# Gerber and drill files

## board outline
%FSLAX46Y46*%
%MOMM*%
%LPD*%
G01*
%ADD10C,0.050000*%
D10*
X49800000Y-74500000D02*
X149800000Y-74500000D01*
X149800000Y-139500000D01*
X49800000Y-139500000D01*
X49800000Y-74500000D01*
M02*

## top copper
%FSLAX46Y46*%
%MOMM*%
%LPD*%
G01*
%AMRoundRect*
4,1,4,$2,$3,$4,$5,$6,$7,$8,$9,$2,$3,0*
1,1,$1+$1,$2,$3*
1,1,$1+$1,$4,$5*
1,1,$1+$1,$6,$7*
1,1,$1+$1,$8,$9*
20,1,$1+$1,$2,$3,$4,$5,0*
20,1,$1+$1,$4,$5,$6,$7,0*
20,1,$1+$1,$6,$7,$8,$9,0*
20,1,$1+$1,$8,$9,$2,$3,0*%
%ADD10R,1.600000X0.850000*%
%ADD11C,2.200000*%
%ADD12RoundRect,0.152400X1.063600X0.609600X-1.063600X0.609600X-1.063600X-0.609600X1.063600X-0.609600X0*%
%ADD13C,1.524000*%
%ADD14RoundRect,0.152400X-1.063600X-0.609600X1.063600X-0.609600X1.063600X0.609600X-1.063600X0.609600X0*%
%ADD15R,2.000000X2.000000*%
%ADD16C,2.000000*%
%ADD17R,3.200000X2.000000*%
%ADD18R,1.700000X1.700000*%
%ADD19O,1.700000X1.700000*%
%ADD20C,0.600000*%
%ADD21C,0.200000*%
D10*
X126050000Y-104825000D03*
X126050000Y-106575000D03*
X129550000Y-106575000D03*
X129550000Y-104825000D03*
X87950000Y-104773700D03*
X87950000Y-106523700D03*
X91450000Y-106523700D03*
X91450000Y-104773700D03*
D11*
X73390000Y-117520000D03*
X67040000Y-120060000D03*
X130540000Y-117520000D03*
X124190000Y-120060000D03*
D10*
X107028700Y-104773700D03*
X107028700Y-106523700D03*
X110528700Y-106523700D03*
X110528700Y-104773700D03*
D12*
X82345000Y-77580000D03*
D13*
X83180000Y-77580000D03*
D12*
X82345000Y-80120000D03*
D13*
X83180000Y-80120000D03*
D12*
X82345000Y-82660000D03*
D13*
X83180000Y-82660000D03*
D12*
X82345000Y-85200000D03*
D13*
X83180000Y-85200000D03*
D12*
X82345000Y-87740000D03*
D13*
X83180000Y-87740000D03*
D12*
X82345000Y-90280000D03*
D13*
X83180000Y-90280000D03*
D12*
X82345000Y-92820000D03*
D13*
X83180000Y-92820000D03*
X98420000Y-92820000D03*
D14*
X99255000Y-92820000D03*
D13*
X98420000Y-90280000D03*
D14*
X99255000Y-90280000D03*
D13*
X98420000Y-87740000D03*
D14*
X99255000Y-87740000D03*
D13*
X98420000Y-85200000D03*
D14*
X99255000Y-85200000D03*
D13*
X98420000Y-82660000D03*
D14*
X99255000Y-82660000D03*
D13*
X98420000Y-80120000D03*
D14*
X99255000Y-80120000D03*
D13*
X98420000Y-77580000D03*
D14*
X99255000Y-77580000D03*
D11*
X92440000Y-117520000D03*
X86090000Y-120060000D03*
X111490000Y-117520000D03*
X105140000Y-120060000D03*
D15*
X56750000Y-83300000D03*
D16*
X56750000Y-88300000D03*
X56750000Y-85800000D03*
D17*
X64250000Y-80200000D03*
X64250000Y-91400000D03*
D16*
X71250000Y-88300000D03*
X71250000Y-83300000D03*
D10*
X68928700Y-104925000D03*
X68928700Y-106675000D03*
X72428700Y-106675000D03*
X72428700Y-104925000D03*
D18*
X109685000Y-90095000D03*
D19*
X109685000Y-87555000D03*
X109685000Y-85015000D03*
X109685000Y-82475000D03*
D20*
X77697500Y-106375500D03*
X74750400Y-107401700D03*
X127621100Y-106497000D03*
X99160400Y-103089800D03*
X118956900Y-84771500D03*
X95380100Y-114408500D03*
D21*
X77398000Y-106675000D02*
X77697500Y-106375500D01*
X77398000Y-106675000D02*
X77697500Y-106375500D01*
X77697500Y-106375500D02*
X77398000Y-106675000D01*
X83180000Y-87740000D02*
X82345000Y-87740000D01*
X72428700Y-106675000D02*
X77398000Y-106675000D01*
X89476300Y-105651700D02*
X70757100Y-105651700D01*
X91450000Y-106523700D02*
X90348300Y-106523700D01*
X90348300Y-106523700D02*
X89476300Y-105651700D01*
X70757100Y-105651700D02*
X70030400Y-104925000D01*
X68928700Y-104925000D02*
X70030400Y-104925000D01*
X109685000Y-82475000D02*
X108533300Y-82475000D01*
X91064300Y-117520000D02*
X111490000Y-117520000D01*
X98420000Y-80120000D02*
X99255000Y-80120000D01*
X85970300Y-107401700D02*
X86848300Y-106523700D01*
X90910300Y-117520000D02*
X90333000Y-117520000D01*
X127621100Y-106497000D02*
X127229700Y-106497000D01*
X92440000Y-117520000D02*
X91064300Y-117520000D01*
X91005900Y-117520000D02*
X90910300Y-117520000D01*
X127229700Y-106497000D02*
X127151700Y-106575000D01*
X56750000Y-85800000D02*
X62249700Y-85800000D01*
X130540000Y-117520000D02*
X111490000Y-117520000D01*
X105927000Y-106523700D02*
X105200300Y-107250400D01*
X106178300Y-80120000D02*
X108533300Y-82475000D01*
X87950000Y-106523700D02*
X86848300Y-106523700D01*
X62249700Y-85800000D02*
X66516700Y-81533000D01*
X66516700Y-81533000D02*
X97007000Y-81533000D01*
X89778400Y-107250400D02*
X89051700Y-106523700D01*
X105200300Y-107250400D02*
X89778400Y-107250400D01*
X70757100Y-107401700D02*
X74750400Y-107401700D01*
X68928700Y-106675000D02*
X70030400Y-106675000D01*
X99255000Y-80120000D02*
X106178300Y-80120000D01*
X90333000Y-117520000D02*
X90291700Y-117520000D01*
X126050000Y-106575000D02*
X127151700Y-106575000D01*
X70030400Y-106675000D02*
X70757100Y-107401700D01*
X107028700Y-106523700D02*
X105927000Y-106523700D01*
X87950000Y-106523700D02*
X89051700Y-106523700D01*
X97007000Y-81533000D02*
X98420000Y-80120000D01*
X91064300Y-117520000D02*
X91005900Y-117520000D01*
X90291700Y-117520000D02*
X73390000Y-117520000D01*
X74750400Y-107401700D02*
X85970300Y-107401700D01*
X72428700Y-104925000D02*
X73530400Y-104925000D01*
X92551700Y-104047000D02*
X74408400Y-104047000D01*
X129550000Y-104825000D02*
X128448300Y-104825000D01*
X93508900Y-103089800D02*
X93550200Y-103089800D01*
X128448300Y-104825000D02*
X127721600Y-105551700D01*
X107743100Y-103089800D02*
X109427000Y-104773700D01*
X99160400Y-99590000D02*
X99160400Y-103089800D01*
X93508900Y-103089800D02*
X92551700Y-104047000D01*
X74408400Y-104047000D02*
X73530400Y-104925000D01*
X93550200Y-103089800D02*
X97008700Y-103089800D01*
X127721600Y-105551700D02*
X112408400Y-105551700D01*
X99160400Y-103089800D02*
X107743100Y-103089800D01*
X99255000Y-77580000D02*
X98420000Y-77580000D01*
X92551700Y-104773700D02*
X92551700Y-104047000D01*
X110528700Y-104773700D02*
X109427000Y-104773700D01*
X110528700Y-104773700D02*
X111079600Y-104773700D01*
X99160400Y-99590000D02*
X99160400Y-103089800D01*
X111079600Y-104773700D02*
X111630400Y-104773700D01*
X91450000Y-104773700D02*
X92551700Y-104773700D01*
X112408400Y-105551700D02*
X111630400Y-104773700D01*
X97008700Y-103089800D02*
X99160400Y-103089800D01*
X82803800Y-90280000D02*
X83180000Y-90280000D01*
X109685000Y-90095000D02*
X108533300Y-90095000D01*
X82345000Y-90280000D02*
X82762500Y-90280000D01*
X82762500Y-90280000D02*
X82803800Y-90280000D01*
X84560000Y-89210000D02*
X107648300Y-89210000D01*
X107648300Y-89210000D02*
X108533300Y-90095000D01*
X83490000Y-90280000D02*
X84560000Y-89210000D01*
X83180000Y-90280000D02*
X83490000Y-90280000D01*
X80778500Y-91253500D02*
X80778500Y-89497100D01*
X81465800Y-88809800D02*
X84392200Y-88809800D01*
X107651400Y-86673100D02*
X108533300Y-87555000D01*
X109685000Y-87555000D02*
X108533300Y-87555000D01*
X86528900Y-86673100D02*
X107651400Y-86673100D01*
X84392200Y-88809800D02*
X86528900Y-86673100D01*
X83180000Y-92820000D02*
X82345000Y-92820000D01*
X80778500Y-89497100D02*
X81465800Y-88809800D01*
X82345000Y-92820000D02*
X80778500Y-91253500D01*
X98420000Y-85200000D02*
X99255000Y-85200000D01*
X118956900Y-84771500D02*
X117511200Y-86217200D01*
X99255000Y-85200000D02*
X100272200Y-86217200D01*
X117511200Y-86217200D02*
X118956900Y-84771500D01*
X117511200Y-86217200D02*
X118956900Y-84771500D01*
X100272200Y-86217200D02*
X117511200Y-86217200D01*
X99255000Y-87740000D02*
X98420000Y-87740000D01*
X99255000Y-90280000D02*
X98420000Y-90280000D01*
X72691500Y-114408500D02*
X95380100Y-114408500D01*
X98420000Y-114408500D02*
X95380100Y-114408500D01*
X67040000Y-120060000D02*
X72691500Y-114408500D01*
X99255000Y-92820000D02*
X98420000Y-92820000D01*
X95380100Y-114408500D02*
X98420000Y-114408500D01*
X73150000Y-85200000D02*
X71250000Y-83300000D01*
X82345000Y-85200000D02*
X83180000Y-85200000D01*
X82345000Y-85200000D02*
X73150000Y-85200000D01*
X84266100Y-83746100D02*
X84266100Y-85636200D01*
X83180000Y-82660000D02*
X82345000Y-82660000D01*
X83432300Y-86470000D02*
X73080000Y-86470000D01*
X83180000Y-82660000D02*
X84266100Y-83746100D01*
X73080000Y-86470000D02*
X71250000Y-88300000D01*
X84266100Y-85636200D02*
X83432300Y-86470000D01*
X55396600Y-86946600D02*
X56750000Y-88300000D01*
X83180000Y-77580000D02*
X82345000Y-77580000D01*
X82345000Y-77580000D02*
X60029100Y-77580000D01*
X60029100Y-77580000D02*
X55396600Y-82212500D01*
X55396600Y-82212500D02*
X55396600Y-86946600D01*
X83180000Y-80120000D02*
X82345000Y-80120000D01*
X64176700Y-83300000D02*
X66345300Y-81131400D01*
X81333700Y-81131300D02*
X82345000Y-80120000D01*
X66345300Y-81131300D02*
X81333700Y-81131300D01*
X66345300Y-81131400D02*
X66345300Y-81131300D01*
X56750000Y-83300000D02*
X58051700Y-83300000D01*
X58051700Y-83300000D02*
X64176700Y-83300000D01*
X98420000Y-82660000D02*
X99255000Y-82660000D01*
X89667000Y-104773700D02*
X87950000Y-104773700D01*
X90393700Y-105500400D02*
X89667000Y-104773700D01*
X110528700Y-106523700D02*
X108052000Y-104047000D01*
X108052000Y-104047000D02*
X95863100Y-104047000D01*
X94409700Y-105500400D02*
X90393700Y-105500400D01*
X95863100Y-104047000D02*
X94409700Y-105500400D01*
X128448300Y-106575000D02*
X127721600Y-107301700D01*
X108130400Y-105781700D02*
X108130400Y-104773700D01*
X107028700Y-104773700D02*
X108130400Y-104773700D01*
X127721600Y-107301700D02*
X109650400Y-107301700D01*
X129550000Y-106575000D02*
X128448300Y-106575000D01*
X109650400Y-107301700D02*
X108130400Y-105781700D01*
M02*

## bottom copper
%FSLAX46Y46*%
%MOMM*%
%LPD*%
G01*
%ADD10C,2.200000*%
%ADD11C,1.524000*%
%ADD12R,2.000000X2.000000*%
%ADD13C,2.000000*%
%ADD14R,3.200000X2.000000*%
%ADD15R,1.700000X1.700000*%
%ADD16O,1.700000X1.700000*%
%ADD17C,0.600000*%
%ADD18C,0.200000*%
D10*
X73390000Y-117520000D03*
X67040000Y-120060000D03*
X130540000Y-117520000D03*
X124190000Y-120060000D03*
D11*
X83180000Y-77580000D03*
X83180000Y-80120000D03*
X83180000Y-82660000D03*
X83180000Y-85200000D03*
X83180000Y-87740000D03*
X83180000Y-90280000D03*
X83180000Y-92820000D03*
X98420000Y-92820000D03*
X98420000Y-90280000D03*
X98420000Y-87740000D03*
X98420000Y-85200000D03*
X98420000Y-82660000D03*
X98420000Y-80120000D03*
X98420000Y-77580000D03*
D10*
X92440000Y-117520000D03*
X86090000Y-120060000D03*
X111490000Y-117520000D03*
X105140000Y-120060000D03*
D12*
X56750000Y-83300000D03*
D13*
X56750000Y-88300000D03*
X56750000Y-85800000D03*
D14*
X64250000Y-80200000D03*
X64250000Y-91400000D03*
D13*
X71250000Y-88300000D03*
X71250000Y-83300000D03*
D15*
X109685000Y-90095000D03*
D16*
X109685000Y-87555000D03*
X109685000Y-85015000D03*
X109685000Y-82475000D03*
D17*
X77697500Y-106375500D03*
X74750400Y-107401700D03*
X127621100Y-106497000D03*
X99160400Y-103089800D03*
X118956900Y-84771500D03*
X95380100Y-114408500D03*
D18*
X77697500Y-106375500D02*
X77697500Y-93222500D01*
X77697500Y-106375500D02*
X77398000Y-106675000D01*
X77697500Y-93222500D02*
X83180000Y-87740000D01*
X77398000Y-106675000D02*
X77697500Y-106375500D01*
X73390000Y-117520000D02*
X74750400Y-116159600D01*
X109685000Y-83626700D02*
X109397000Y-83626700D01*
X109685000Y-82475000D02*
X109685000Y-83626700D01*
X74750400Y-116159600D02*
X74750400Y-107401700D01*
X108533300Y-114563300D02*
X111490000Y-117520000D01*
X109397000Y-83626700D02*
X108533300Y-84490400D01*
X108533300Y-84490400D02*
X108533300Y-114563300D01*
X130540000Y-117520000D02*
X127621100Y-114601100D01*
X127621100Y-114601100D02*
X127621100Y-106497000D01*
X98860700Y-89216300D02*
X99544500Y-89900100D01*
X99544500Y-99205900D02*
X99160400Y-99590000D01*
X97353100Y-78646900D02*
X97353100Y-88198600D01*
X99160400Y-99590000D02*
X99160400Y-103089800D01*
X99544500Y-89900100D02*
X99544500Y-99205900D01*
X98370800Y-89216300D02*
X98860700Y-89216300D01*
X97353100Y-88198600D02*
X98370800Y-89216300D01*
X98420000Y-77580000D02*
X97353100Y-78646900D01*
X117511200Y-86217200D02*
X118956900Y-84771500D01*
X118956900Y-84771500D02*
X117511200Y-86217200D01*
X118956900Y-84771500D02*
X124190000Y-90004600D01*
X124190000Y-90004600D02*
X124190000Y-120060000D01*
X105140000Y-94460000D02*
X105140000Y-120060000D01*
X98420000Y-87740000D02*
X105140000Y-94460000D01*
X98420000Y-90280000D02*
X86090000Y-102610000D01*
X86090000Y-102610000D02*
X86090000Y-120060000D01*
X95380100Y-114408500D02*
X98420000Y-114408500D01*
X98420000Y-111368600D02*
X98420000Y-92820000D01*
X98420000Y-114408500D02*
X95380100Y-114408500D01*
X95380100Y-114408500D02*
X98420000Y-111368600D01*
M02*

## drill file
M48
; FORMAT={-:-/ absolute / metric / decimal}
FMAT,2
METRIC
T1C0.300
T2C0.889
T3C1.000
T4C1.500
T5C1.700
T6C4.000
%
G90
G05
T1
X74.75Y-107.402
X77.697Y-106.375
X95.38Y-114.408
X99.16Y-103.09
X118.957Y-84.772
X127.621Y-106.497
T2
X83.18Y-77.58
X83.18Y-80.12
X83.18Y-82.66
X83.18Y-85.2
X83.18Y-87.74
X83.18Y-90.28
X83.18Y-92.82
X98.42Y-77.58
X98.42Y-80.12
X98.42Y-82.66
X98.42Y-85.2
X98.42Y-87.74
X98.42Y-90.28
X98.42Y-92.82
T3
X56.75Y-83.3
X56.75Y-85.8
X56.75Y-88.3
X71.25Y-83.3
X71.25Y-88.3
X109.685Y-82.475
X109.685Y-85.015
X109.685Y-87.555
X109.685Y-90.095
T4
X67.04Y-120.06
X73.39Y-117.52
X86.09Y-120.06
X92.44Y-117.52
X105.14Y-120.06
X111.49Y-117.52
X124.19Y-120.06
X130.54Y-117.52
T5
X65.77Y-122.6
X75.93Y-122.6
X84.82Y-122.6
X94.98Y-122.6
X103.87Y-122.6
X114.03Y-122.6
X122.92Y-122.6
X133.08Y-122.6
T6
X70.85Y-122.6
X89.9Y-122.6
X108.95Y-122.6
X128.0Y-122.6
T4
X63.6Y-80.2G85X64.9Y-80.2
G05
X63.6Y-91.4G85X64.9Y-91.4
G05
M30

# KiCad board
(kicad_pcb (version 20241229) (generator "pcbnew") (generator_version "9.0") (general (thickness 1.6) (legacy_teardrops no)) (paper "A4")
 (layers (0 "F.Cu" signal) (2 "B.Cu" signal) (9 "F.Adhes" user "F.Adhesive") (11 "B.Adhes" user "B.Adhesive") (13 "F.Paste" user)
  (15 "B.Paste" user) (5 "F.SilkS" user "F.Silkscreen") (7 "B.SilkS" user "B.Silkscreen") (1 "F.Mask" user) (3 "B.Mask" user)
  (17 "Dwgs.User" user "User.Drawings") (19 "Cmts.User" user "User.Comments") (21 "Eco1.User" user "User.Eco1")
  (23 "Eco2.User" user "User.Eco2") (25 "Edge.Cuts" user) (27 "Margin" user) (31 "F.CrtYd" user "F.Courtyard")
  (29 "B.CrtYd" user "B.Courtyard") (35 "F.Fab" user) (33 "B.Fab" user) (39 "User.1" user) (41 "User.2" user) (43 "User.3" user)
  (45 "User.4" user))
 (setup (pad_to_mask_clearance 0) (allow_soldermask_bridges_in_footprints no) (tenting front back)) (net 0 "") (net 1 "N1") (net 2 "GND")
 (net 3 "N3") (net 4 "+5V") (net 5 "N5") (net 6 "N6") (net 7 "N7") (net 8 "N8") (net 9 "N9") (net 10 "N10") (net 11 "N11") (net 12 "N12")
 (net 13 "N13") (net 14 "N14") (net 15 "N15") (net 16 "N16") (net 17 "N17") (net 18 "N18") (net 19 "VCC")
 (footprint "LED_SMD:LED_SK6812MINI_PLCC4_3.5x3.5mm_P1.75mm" (layer "F.Cu") (at 127.8 105.7)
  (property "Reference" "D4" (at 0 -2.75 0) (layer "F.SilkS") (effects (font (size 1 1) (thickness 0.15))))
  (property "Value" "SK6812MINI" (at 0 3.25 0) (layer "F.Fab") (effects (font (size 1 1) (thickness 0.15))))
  (pad "1" smd rect (at -1.75 -0.875) (size 1.6 0.85) (layers "F.Cu" "F.Mask" "F.Paste") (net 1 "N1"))
  (pad "2" smd rect (at -1.75 0.875) (size 1.6 0.85) (layers "F.Cu" "F.Mask" "F.Paste") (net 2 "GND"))
  (pad "3" smd rect (at 1.75 0.875) (size 1.6 0.85) (layers "F.Cu" "F.Mask" "F.Paste") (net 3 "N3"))
  (pad "4" smd rect (at 1.75 -0.875) (size 1.6 0.85) (layers "F.Cu" "F.Mask" "F.Paste") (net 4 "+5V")))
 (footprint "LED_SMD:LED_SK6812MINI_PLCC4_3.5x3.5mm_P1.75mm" (layer "F.Cu") (at 89.7 105.6487)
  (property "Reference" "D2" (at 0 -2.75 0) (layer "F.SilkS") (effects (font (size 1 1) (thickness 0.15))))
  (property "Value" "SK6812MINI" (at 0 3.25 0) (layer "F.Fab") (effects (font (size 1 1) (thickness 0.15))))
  (pad "1" smd rect (at -1.75 -0.875) (size 1.6 0.85) (layers "F.Cu" "F.Mask" "F.Paste") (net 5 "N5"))
  (pad "2" smd rect (at -1.75 0.875) (size 1.6 0.85) (layers "F.Cu" "F.Mask" "F.Paste") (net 2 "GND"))
  (pad "3" smd rect (at 1.75 0.875) (size 1.6 0.85) (layers "F.Cu" "F.Mask" "F.Paste") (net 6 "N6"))
  (pad "4" smd rect (at 1.75 -0.875) (size 1.6 0.85) (layers "F.Cu" "F.Mask" "F.Paste") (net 4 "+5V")))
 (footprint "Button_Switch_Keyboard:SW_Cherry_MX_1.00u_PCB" (layer "F.Cu") (at 73.39 117.52)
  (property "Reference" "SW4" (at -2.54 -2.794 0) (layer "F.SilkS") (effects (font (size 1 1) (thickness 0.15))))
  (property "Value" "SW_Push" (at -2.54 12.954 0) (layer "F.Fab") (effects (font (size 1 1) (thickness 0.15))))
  (pad "" np_thru_hole circle (at -7.62 5.08) (size 1.7 1.7) (drill 1.7) (layers "*.Cu" "*.Mask"))
  (pad "" np_thru_hole circle (at -2.54 5.08) (size 4 4) (drill 4) (layers "*.Cu" "*.Mask"))
  (pad "" np_thru_hole circle (at 2.54 5.08) (size 1.7 1.7) (drill 1.7) (layers "*.Cu" "*.Mask"))
  (pad "1" thru_hole circle (at 0 0) (size 2.2 2.2) (drill 1.5) (layers "*.Cu" "*.Mask") (remove_unused_layers no) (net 2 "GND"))
  (pad "2" thru_hole circle (at -6.35 2.54) (size 2.2 2.2) (drill 1.5) (layers "*.Cu" "*.Mask") (remove_unused_layers no) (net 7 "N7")))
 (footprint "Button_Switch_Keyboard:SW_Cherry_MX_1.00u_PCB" (layer "F.Cu") (at 130.54 117.52)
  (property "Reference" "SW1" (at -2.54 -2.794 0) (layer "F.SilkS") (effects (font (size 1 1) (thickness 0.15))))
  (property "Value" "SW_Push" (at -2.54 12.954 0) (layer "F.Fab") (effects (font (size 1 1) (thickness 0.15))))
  (pad "" np_thru_hole circle (at -7.62 5.08) (size 1.7 1.7) (drill 1.7) (layers "*.Cu" "*.Mask"))
  (pad "" np_thru_hole circle (at -2.54 5.08) (size 4 4) (drill 4) (layers "*.Cu" "*.Mask"))
  (pad "" np_thru_hole circle (at 2.54 5.08) (size 1.7 1.7) (drill 1.7) (layers "*.Cu" "*.Mask"))
  (pad "1" thru_hole circle (at 0 0) (size 2.2 2.2) (drill 1.5) (layers "*.Cu" "*.Mask") (remove_unused_layers no) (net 2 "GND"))
  (pad "2" thru_hole circle (at -6.35 2.54) (size 2.2 2.2) (drill 1.5) (layers "*.Cu" "*.Mask") (remove_unused_layers no) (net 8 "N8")))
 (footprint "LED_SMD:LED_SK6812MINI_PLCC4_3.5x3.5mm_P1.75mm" (layer "F.Cu") (at 108.7787 105.6487)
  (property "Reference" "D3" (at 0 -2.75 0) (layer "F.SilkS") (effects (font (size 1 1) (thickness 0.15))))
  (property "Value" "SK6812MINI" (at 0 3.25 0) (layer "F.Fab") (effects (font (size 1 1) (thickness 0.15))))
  (pad "1" smd rect (at -1.75 -0.875) (size 1.6 0.85) (layers "F.Cu" "F.Mask" "F.Paste") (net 3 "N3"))
  (pad "2" smd rect (at -1.75 0.875) (size 1.6 0.85) (layers "F.Cu" "F.Mask" "F.Paste") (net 2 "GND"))
  (pad "3" smd rect (at 1.75 0.875) (size 1.6 0.85) (layers "F.Cu" "F.Mask" "F.Paste") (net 5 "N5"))
  (pad "4" smd rect (at 1.75 -0.875) (size 1.6 0.85) (layers "F.Cu" "F.Mask" "F.Paste") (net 4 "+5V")))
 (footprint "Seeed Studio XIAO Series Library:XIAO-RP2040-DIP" (layer "F.Cu") (at 90.8 85.2)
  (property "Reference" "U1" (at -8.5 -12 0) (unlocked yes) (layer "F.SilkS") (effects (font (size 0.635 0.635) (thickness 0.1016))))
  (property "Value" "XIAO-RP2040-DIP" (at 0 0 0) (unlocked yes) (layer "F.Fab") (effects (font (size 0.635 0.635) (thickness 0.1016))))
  (pad "1" smd roundrect (at -8.455 -7.62 180) (size 2.432 1.524) (layers "F.Cu" "F.Mask") (roundrect_rratio 0.1) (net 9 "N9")
   (thermal_bridge_angle 45))
  (pad "1" thru_hole circle (at -7.62 -7.62 180) (size 1.524 1.524) (drill 0.889) (layers "*.Cu" "*.Mask") (remove_unused_layers no)
   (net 9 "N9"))
  (pad "2" smd roundrect (at -8.455 -5.08 180) (size 2.432 1.524) (layers "F.Cu" "F.Mask") (roundrect_rratio 0.1) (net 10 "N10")
   (thermal_bridge_angle 45))
  (pad "2" thru_hole circle (at -7.62 -5.08 180) (size 1.524 1.524) (drill 0.889) (layers "*.Cu" "*.Mask") (remove_unused_layers no)
   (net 10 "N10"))
  (pad "3" smd roundrect (at -8.455 -2.54 180) (size 2.432 1.524) (layers "F.Cu" "F.Mask") (roundrect_rratio 0.1) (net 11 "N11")
   (thermal_bridge_angle 45))
  (pad "3" thru_hole circle (at -7.62 -2.54 180) (size 1.524 1.524) (drill 0.889) (layers "*.Cu" "*.Mask") (remove_unused_layers no)
   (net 11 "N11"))
  (pad "4" smd roundrect (at -8.455 0 180) (size 2.432 1.524) (layers "F.Cu" "F.Mask") (roundrect_rratio 0.1) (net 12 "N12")
   (thermal_bridge_angle 45))
  (pad "4" thru_hole circle (at -7.62 0 180) (size 1.524 1.524) (drill 0.889) (layers "*.Cu" "*.Mask") (remove_unused_layers no)
   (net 12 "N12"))
  (pad "5" smd roundrect (at -8.455 2.54 180) (size 2.432 1.524) (layers "F.Cu" "F.Mask") (roundrect_rratio 0.1) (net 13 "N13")
   (thermal_bridge_angle 45))
  (pad "5" thru_hole circle (at -7.62 2.54 180) (size 1.524 1.524) (drill 0.889) (layers "*.Cu" "*.Mask") (remove_unused_layers no)
   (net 13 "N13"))
  (pad "6" smd roundrect (at -8.455 5.08 180) (size 2.432 1.524) (layers "F.Cu" "F.Mask") (roundrect_rratio 0.1) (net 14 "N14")
   (thermal_bridge_angle 45))
  (pad "6" thru_hole circle (at -7.62 5.08 180) (size 1.524 1.524) (drill 0.889) (layers "*.Cu" "*.Mask") (remove_unused_layers no)
   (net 14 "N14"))
  (pad "7" smd roundrect (at -8.455 7.62 180) (size 2.432 1.524) (layers "F.Cu" "F.Mask") (roundrect_rratio 0.1) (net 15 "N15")
   (thermal_bridge_angle 45))
  (pad "7" thru_hole circle (at -7.62 7.62 180) (size 1.524 1.524) (drill 0.889) (layers "*.Cu" "*.Mask") (remove_unused_layers no)
   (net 15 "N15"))
  (pad "8" thru_hole circle (at 7.62 7.62) (size 1.524 1.524) (drill 0.889) (layers "*.Cu" "*.Mask") (remove_unused_layers no) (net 7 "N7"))
  (pad "8" smd roundrect (at 8.455 7.62) (size 2.432 1.524) (layers "F.Cu" "F.Mask") (roundrect_rratio 0.1) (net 7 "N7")
   (thermal_bridge_angle 45))
  (pad "9" thru_hole circle (at 7.62 5.08) (size 1.524 1.524) (drill 0.889) (layers "*.Cu" "*.Mask") (remove_unused_layers no)
   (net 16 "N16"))
  (pad "9" smd roundrect (at 8.455 5.08) (size 2.432 1.524) (layers "F.Cu" "F.Mask") (roundrect_rratio 0.1) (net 16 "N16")
   (thermal_bridge_angle 45))
  (pad "10" thru_hole circle (at 7.62 2.54) (size 1.524 1.524) (drill 0.889) (layers "*.Cu" "*.Mask") (remove_unused_layers no)
   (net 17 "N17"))
  (pad "10" smd roundrect (at 8.455 2.54) (size 2.432 1.524) (layers "F.Cu" "F.Mask") (roundrect_rratio 0.1) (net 17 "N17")
   (thermal_bridge_angle 45))
  (pad "11" thru_hole circle (at 7.62 0) (size 1.524 1.524) (drill 0.889) (layers "*.Cu" "*.Mask") (remove_unused_layers no) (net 8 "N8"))
  (pad "11" smd roundrect (at 8.455 0) (size 2.432 1.524) (layers "F.Cu" "F.Mask") (roundrect_rratio 0.1) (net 8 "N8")
   (thermal_bridge_angle 45))
  (pad "12" thru_hole circle (at 7.62 -2.54) (size 1.524 1.524) (drill 0.889) (layers "*.Cu" "*.Mask") (remove_unused_layers no)
   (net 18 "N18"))
  (pad "12" smd roundrect (at 8.455 -2.54) (size 2.432 1.524) (layers "F.Cu" "F.Mask") (roundrect_rratio 0.1) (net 18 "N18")
   (thermal_bridge_angle 45))
  (pad "13" thru_hole circle (at 7.62 -5.08) (size 1.524 1.524) (drill 0.889) (layers "*.Cu" "*.Mask") (remove_unused_layers no)
   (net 2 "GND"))
  (pad "13" smd roundrect (at 8.455 -5.08) (size 2.432 1.524) (layers "F.Cu" "F.Mask") (roundrect_rratio 0.1) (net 2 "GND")
   (thermal_bridge_angle 45))
  (pad "14" thru_hole circle (at 7.62 -7.62) (size 1.524 1.524) (drill 0.889) (layers "*.Cu" "*.Mask") (remove_unused_layers no)
   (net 4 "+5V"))
  (pad "14" smd roundrect (at 8.455 -7.62) (size 2.432 1.524) (layers "F.Cu" "F.Mask") (roundrect_rratio 0.1) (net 4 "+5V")
   (thermal_bridge_angle 45)))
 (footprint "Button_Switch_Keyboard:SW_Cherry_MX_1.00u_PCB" (layer "F.Cu") (at 92.44 117.52)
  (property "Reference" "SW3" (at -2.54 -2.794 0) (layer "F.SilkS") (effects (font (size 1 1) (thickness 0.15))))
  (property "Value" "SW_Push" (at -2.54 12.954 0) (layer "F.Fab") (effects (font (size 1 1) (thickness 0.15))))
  (pad "" np_thru_hole circle (at -7.62 5.08) (size 1.7 1.7) (drill 1.7) (layers "*.Cu" "*.Mask"))
  (pad "" np_thru_hole circle (at -2.54 5.08) (size 4 4) (drill 4) (layers "*.Cu" "*.Mask"))
  (pad "" np_thru_hole circle (at 2.54 5.08) (size 1.7 1.7) (drill 1.7) (layers "*.Cu" "*.Mask"))
  (pad "1" thru_hole circle (at 0 0) (size 2.2 2.2) (drill 1.5) (layers "*.Cu" "*.Mask") (remove_unused_layers no) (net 2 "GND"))
  (pad "2" thru_hole circle (at -6.35 2.54) (size 2.2 2.2) (drill 1.5) (layers "*.Cu" "*.Mask") (remove_unused_layers no) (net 16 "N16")))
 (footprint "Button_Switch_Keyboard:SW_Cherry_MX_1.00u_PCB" (layer "F.Cu") (at 111.49 117.52)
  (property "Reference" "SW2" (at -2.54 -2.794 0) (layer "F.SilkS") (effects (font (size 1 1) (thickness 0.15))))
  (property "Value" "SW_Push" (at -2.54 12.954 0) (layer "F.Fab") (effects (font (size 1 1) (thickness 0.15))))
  (pad "" np_thru_hole circle (at -7.62 5.08) (size 1.7 1.7) (drill 1.7) (layers "*.Cu" "*.Mask"))
  (pad "" np_thru_hole circle (at -2.54 5.08) (size 4 4) (drill 4) (layers "*.Cu" "*.Mask"))
  (pad "" np_thru_hole circle (at 2.54 5.08) (size 1.7 1.7) (drill 1.7) (layers "*.Cu" "*.Mask"))
  (pad "1" thru_hole circle (at 0 0) (size 2.2 2.2) (drill 1.5) (layers "*.Cu" "*.Mask") (remove_unused_layers no) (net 2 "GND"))
  (pad "2" thru_hole circle (at -6.35 2.54) (size 2.2 2.2) (drill 1.5) (layers "*.Cu" "*.Mask") (remove_unused_layers no) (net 17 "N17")))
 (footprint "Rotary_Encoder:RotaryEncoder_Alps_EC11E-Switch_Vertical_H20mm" (layer "F.Cu") (at 56.75 83.3)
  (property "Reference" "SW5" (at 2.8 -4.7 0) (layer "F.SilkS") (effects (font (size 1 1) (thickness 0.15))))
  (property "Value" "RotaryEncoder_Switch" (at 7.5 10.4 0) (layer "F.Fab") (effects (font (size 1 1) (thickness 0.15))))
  (pad "A" thru_hole rect (at 0 0) (size 2 2) (drill 1) (layers "*.Cu" "*.Mask") (remove_unused_layers no) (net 10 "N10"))
  (pad "B" thru_hole circle (at 0 5) (size 2 2) (drill 1) (layers "*.Cu" "*.Mask") (remove_unused_layers no) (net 9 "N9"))
  (pad "C" thru_hole circle (at 0 2.5) (size 2 2) (drill 1) (layers "*.Cu" "*.Mask") (remove_unused_layers no) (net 2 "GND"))
  (pad "MP" thru_hole rect (at 7.5 -3.1) (size 3.2 2) (drill oval 2.8 1.5) (layers "*.Cu" "*.Mask") (remove_unused_layers no))
  (pad "MP" thru_hole rect (at 7.5 8.1) (size 3.2 2) (drill oval 2.8 1.5) (layers "*.Cu" "*.Mask") (remove_unused_layers no))
  (pad "S1" thru_hole circle (at 14.5 5) (size 2 2) (drill 1) (layers "*.Cu" "*.Mask") (remove_unused_layers no) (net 11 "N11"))
  (pad "S2" thru_hole circle (at 14.5 0) (size 2 2) (drill 1) (layers "*.Cu" "*.Mask") (remove_unused_layers no) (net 12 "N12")))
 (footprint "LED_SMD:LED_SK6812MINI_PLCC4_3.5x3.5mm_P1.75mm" (layer "F.Cu") (at 70.6787 105.8)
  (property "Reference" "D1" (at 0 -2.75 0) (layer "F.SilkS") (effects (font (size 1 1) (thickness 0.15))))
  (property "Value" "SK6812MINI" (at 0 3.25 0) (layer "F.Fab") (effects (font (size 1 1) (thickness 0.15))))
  (pad "1" smd rect (at -1.75 -0.875) (size 1.6 0.85) (layers "F.Cu" "F.Mask" "F.Paste") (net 6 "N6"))
  (pad "2" smd rect (at -1.75 0.875) (size 1.6 0.85) (layers "F.Cu" "F.Mask" "F.Paste") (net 2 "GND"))
  (pad "3" smd rect (at 1.75 0.875) (size 1.6 0.85) (layers "F.Cu" "F.Mask" "F.Paste") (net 13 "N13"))
  (pad "4" smd rect (at 1.75 -0.875) (size 1.6 0.85) (layers "F.Cu" "F.Mask" "F.Paste") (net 4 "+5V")))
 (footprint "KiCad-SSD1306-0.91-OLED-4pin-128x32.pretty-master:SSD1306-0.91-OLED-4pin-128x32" (layer "F.Cu") (at 146.185 92.285 180)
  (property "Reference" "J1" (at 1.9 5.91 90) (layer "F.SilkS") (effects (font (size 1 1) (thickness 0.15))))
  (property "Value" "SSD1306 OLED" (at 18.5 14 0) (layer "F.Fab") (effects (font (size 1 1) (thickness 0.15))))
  (pad "1" thru_hole rect (at 36.5 2.19 180) (size 1.7 1.7) (drill 1) (layers "*.Cu" "*.Mask") (remove_unused_layers no) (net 14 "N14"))
  (pad "2" thru_hole oval (at 36.5 4.73 180) (size 1.7 1.7) (drill 1) (layers "*.Cu" "*.Mask") (remove_unused_layers no) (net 15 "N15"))
  (pad "3" thru_hole oval (at 36.5 7.27 180) (size 1.7 1.7) (drill 1) (layers "*.Cu" "*.Mask") (remove_unused_layers no) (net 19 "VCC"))
  (pad "4" thru_hole oval (at 36.5 9.81 180) (size 1.7 1.7) (drill 1) (layers "*.Cu" "*.Mask") (remove_unused_layers no) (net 2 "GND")))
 (gr_rect (start 49.8 74.5) (end 149.8 139.5) (stroke (width 0.05) (type default)) (fill no) (layer "Edge.Cuts"))
 (segment (start 77.398 106.675) (end 77.6975 106.3755) (width 0.2) (layer "F.Cu") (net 13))
 (segment (start 77.398 106.675) (end 77.6975 106.3755) (width 0.2) (layer "F.Cu") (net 13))
 (segment (start 77.6975 106.3755) (end 77.398 106.675) (width 0.2) (layer "F.Cu") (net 13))
 (segment (start 83.18 87.74) (end 82.345 87.74) (width 0.2) (layer "F.Cu") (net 13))
 (segment (start 72.4287 106.675) (end 77.398 106.675) (width 0.2) (layer "F.Cu") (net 13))
 (via (at 77.6975 106.3755) (size 0.6) (drill 0.3) (layers "F.Cu" "B.Cu") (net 13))
 (segment (start 77.6975 106.3755) (end 77.6975 93.2225) (width 0.2) (layer "B.Cu") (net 13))
 (segment (start 77.6975 106.3755) (end 77.398 106.675) (width 0.2) (layer "B.Cu") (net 13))
 (segment (start 77.6975 93.2225) (end 83.18 87.74) (width 0.2) (layer "B.Cu") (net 13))
 (segment (start 77.398 106.675) (end 77.6975 106.3755) (width 0.2) (layer "B.Cu") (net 13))
 (segment (start 89.4763 105.6517) (end 70.7571 105.6517) (width 0.2) (layer "F.Cu") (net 6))
 (segment (start 91.45 106.5237) (end 90.3483 106.5237) (width 0.2) (layer "F.Cu") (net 6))
 (segment (start 90.3483 106.5237) (end 89.4763 105.6517) (width 0.2) (layer "F.Cu") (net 6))
 (segment (start 70.7571 105.6517) (end 70.0304 104.925) (width 0.2) (layer "F.Cu") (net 6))
 (segment (start 68.9287 104.925) (end 70.0304 104.925) (width 0.2) (layer "F.Cu") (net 6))
 (segment (start 109.685 82.475) (end 108.5333 82.475) (width 0.2) (layer "F.Cu") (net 2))
 (segment (start 91.0643 117.52) (end 111.49 117.52) (width 0.2) (layer "F.Cu") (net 2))
 (segment (start 98.42 80.12) (end 99.255 80.12) (width 0.2) (layer "F.Cu") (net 2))
 (segment (start 85.9703 107.4017) (end 86.8483 106.5237) (width 0.2) (layer "F.Cu") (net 2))
 (segment (start 90.9103 117.52) (end 90.333 117.52) (width 0.2) (layer "F.Cu") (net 2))
 (segment (start 127.6211 106.497) (end 127.2297 106.497) (width 0.2) (layer "F.Cu") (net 2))
 (segment (start 92.44 117.52) (end 91.0643 117.52) (width 0.2) (layer "F.Cu") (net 2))
 (segment (start 91.0059 117.52) (end 90.9103 117.52) (width 0.2) (layer "F.Cu") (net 2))
 (segment (start 127.2297 106.497) (end 127.1517 106.575) (width 0.2) (layer "F.Cu") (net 2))
 (segment (start 56.75 85.8) (end 62.2497 85.8) (width 0.2) (layer "F.Cu") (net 2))
 (segment (start 130.54 117.52) (end 111.49 117.52) (width 0.2) (layer "F.Cu") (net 2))
 (segment (start 105.927 106.5237) (end 105.2003 107.2504) (width 0.2) (layer "F.Cu") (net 2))
 (segment (start 106.1783 80.12) (end 108.5333 82.475) (width 0.2) (layer "F.Cu") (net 2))
 (segment (start 87.95 106.5237) (end 86.8483 106.5237) (width 0.2) (layer "F.Cu") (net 2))
 (segment (start 62.2497 85.8) (end 66.5167 81.533) (width 0.2) (layer "F.Cu") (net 2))
 (segment (start 66.5167 81.533) (end 97.007 81.533) (width 0.2) (layer "F.Cu") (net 2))
 (segment (start 89.7784 107.2504) (end 89.0517 106.5237) (width 0.2) (layer "F.Cu") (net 2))
 (segment (start 105.2003 107.2504) (end 89.7784 107.2504) (width 0.2) (layer "F.Cu") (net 2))
 (segment (start 70.7571 107.4017) (end 74.7504 107.4017) (width 0.2) (layer "F.Cu") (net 2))
 (segment (start 68.9287 106.675) (end 70.0304 106.675) (width 0.2) (layer "F.Cu") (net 2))
 (segment (start 99.255 80.12) (end 106.1783 80.12) (width 0.2) (layer "F.Cu") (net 2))
 (segment (start 90.333 117.52) (end 90.2917 117.52) (width 0.2) (layer "F.Cu") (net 2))
 (segment (start 126.05 106.575) (end 127.1517 106.575) (width 0.2) (layer "F.Cu") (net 2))
 (segment (start 70.0304 106.675) (end 70.7571 107.4017) (width 0.2) (layer "F.Cu") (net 2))
 (segment (start 107.0287 106.5237) (end 105.927 106.5237) (width 0.2) (layer "F.Cu") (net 2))
 (segment (start 87.95 106.5237) (end 89.0517 106.5237) (width 0.2) (layer "F.Cu") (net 2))
 (segment (start 97.007 81.533) (end 98.42 80.12) (width 0.2) (layer "F.Cu") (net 2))
 (segment (start 91.0643 117.52) (end 91.0059 117.52) (width 0.2) (layer "F.Cu") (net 2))
 (segment (start 90.2917 117.52) (end 73.39 117.52) (width 0.2) (layer "F.Cu") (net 2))
 (segment (start 74.7504 107.4017) (end 85.9703 107.4017) (width 0.2) (layer "F.Cu") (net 2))
 (via (at 74.7504 107.4017) (size 0.6) (drill 0.3) (layers "F.Cu" "B.Cu") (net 2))
 (via (at 127.6211 106.497) (size 0.6) (drill 0.3) (layers "F.Cu" "B.Cu") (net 2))
 (segment (start 73.39 117.52) (end 74.7504 116.1596) (width 0.2) (layer "B.Cu") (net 2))
 (segment (start 109.685 83.6267) (end 109.397 83.6267) (width 0.2) (layer "B.Cu") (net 2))
 (segment (start 109.685 82.475) (end 109.685 83.6267) (width 0.2) (layer "B.Cu") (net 2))
 (segment (start 74.7504 116.1596) (end 74.7504 107.4017) (width 0.2) (layer "B.Cu") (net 2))
 (segment (start 108.5333 114.5633) (end 111.49 117.52) (width 0.2) (layer "B.Cu") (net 2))
 (segment (start 109.397 83.6267) (end 108.5333 84.4904) (width 0.2) (layer "B.Cu") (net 2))
 (segment (start 108.5333 84.4904) (end 108.5333 114.5633) (width 0.2) (layer "B.Cu") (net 2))
 (segment (start 130.54 117.52) (end 127.6211 114.6011) (width 0.2) (layer "B.Cu") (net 2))
 (segment (start 127.6211 114.6011) (end 127.6211 106.497) (width 0.2) (layer "B.Cu") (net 2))
 (segment (start 72.4287 104.925) (end 73.5304 104.925) (width 0.2) (layer "F.Cu") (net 4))
 (segment (start 92.5517 104.047) (end 74.4084 104.047) (width 0.2) (layer "F.Cu") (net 4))
 (segment (start 129.55 104.825) (end 128.4483 104.825) (width 0.2) (layer "F.Cu") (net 4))
 (segment (start 93.5089 103.0898) (end 93.5502 103.0898) (width 0.2) (layer "F.Cu") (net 4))
 (segment (start 128.4483 104.825) (end 127.7216 105.5517) (width 0.2) (layer "F.Cu") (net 4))
 (segment (start 107.7431 103.0898) (end 109.427 104.7737) (width 0.2) (layer "F.Cu") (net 4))
 (segment (start 99.1604 99.59) (end 99.1604 103.0898) (width 0.2) (layer "F.Cu") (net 4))
 (segment (start 93.5089 103.0898) (end 92.5517 104.047) (width 0.2) (layer "F.Cu") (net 4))
 (segment (start 74.4084 104.047) (end 73.5304 104.925) (width 0.2) (layer "F.Cu") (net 4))
 (segment (start 93.5502 103.0898) (end 97.0087 103.0898) (width 0.2) (layer "F.Cu") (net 4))
 (segment (start 127.7216 105.5517) (end 112.4084 105.5517) (width 0.2) (layer "F.Cu") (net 4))
 (segment (start 99.1604 103.0898) (end 107.7431 103.0898) (width 0.2) (layer "F.Cu") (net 4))
 (segment (start 99.255 77.58) (end 98.42 77.58) (width 0.2) (layer "F.Cu") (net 4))
 (segment (start 92.5517 104.7737) (end 92.5517 104.047) (width 0.2) (layer "F.Cu") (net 4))
 (segment (start 110.5287 104.7737) (end 109.427 104.7737) (width 0.2) (layer "F.Cu") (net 4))
 (segment (start 110.5287 104.7737) (end 111.0796 104.7737) (width 0.2) (layer "F.Cu") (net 4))
 (segment (start 99.1604 99.59) (end 99.1604 103.0898) (width 0.2) (layer "F.Cu") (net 4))
 (segment (start 111.0796 104.7737) (end 111.6304 104.7737) (width 0.2) (layer "F.Cu") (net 4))
 (segment (start 91.45 104.7737) (end 92.5517 104.7737) (width 0.2) (layer "F.Cu") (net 4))
 (segment (start 112.4084 105.5517) (end 111.6304 104.7737) (width 0.2) (layer "F.Cu") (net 4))
 (segment (start 97.0087 103.0898) (end 99.1604 103.0898) (width 0.2) (layer "F.Cu") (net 4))
 (via (at 99.1604 103.0898) (size 0.6) (drill 0.3) (layers "F.Cu" "B.Cu") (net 4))
 (segment (start 98.8607 89.2163) (end 99.5445 89.9001) (width 0.2) (layer "B.Cu") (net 4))
 (segment (start 99.5445 99.2059) (end 99.1604 99.59) (width 0.2) (layer "B.Cu") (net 4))
 (segment (start 97.3531 78.6469) (end 97.3531 88.1986) (width 0.2) (layer "B.Cu") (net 4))
 (segment (start 99.1604 99.59) (end 99.1604 103.0898) (width 0.2) (layer "B.Cu") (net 4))
 (segment (start 99.5445 89.9001) (end 99.5445 99.2059) (width 0.2) (layer "B.Cu") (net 4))
 (segment (start 98.3708 89.2163) (end 98.8607 89.2163) (width 0.2) (layer "B.Cu") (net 4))
 (segment (start 97.3531 88.1986) (end 98.3708 89.2163) (width 0.2) (layer "B.Cu") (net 4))
 (segment (start 98.42 77.58) (end 97.3531 78.6469) (width 0.2) (layer "B.Cu") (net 4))
 (segment (start 82.8038 90.28) (end 83.18 90.28) (width 0.2) (layer "F.Cu") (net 14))
 (segment (start 109.685 90.095) (end 108.5333 90.095) (width 0.2) (layer "F.Cu") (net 14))
 (segment (start 82.345 90.28) (end 82.7625 90.28) (width 0.2) (layer "F.Cu") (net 14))
 (segment (start 82.7625 90.28) (end 82.8038 90.28) (width 0.2) (layer "F.Cu") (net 14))
 (segment (start 84.56 89.21) (end 107.6483 89.21) (width 0.2) (layer "F.Cu") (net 14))
 (segment (start 107.6483 89.21) (end 108.5333 90.095) (width 0.2) (layer "F.Cu") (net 14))
 (segment (start 83.49 90.28) (end 84.56 89.21) (width 0.2) (layer "F.Cu") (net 14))
 (segment (start 83.18 90.28) (end 83.49 90.28) (width 0.2) (layer "F.Cu") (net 14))
 (segment (start 80.7785 91.2535) (end 80.7785 89.4971) (width 0.2) (layer "F.Cu") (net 15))
 (segment (start 81.4658 88.8098) (end 84.3922 88.8098) (width 0.2) (layer "F.Cu") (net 15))
 (segment (start 107.6514 86.6731) (end 108.5333 87.555) (width 0.2) (layer "F.Cu") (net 15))
 (segment (start 109.685 87.555) (end 108.5333 87.555) (width 0.2) (layer "F.Cu") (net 15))
 (segment (start 86.5289 86.6731) (end 107.6514 86.6731) (width 0.2) (layer "F.Cu") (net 15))
 (segment (start 84.3922 88.8098) (end 86.5289 86.6731) (width 0.2) (layer "F.Cu") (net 15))
 (segment (start 83.18 92.82) (end 82.345 92.82) (width 0.2) (layer "F.Cu") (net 15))
 (segment (start 80.7785 89.4971) (end 81.4658 88.8098) (width 0.2) (layer "F.Cu") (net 15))
 (segment (start 82.345 92.82) (end 80.7785 91.2535) (width 0.2) (layer "F.Cu") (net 15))
 (segment (start 98.42 85.2) (end 99.255 85.2) (width 0.2) (layer "F.Cu") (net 8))
 (segment (start 118.9569 84.7715) (end 117.5112 86.2172) (width 0.2) (layer "F.Cu") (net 8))
 (segment (start 99.255 85.2) (end 100.2722 86.2172) (width 0.2) (layer "F.Cu") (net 8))
 (segment (start 117.5112 86.2172) (end 118.9569 84.7715) (width 0.2) (layer "F.Cu") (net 8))
 (segment (start 117.5112 86.2172) (end 118.9569 84.7715) (width 0.2) (layer "F.Cu") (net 8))
 (segment (start 100.2722 86.2172) (end 117.5112 86.2172) (width 0.2) (layer "F.Cu") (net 8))
 (via (at 118.9569 84.7715) (size 0.6) (drill 0.3) (layers "F.Cu" "B.Cu") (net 8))
 (segment (start 117.5112 86.2172) (end 118.9569 84.7715) (width 0.2) (layer "B.Cu") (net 8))
 (segment (start 118.9569 84.7715) (end 117.5112 86.2172) (width 0.2) (layer "B.Cu") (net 8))
 (segment (start 118.9569 84.7715) (end 124.19 90.0046) (width 0.2) (layer "B.Cu") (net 8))
 (segment (start 124.19 90.0046) (end 124.19 120.06) (width 0.2) (layer "B.Cu") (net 8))
 (segment (start 99.255 87.74) (end 98.42 87.74) (width 0.2) (layer "F.Cu") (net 17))
 (segment (start 105.14 94.46) (end 105.14 120.06) (width 0.2) (layer "B.Cu") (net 17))
 (segment (start 98.42 87.74) (end 105.14 94.46) (width 0.2) (layer "B.Cu") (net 17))
 (segment (start 99.255 90.28) (end 98.42 90.28) (width 0.2) (layer "F.Cu") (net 16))
 (segment (start 98.42 90.28) (end 86.09 102.61) (width 0.2) (layer "B.Cu") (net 16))
 (segment (start 86.09 102.61) (end 86.09 120.06) (width 0.2) (layer "B.Cu") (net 16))
 (segment (start 72.6915 114.4085) (end 95.3801 114.4085) (width 0.2) (layer "F.Cu") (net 7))
 (segment (start 98.42 114.4085) (end 95.3801 114.4085) (width 0.2) (layer "F.Cu") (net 7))
 (segment (start 67.04 120.06) (end 72.6915 114.4085) (width 0.2) (layer "F.Cu") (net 7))
 (segment (start 99.255 92.82) (end 98.42 92.82) (width 0.2) (layer "F.Cu") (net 7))
 (segment (start 95.3801 114.4085) (end 98.42 114.4085) (width 0.2) (layer "F.Cu") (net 7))
 (via (at 95.3801 114.4085) (size 0.6) (drill 0.3) (layers "F.Cu" "B.Cu") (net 7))
 (segment (start 95.3801 114.4085) (end 98.42 114.4085) (width 0.2) (layer "B.Cu") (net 7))
 (segment (start 98.42 111.3686) (end 98.42 92.82) (width 0.2) (layer "B.Cu") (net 7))
 (segment (start 98.42 114.4085) (end 95.3801 114.4085) (width 0.2) (layer "B.Cu") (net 7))
 (segment (start 95.3801 114.4085) (end 98.42 111.3686) (width 0.2) (layer "B.Cu") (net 7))
 (segment (start 73.15 85.2) (end 71.25 83.3) (width 0.2) (layer "F.Cu") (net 12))
 (segment (start 82.345 85.2) (end 83.18 85.2) (width 0.2) (layer "F.Cu") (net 12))
 (segment (start 82.345 85.2) (end 73.15 85.2) (width 0.2) (layer "F.Cu") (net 12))
 (segment (start 84.2661 83.7461) (end 84.2661 85.6362) (width 0.2) (layer "F.Cu") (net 11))
 (segment (start 83.18 82.66) (end 82.345 82.66) (width 0.2) (layer "F.Cu") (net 11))
 (segment (start 83.4323 86.47) (end 73.08 86.47) (width 0.2) (layer "F.Cu") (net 11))
 (segment (start 83.18 82.66) (end 84.2661 83.7461) (width 0.2) (layer "F.Cu") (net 11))
 (segment (start 73.08 86.47) (end 71.25 88.3) (width 0.2) (layer "F.Cu") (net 11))
 (segment (start 84.2661 85.6362) (end 83.4323 86.47) (width 0.2) (layer "F.Cu") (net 11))
 (segment (start 55.3966 86.9466) (end 56.75 88.3) (width 0.2) (layer "F.Cu") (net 9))
 (segment (start 83.18 77.58) (end 82.345 77.58) (width 0.2) (layer "F.Cu") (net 9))
 (segment (start 82.345 77.58) (end 60.0291 77.58) (width 0.2) (layer "F.Cu") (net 9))
 (segment (start 60.0291 77.58) (end 55.3966 82.2125) (width 0.2) (layer "F.Cu") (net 9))
 (segment (start 55.3966 82.2125) (end 55.3966 86.9466) (width 0.2) (layer "F.Cu") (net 9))
 (segment (start 83.18 80.12) (end 82.345 80.12) (width 0.2) (layer "F.Cu") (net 10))
 (segment (start 64.1767 83.3) (end 66.3453 81.1314) (width 0.2) (layer "F.Cu") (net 10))
 (segment (start 81.3337 81.1313) (end 82.345 80.12) (width 0.2) (layer "F.Cu") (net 10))
 (segment (start 66.3453 81.1313) (end 81.3337 81.1313) (width 0.2) (layer "F.Cu") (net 10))
 (segment (start 66.3453 81.1314) (end 66.3453 81.1313) (width 0.2) (layer "F.Cu") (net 10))
 (segment (start 56.75 83.3) (end 58.0517 83.3) (width 0.2) (layer "F.Cu") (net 10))
 (segment (start 58.0517 83.3) (end 64.1767 83.3) (width 0.2) (layer "F.Cu") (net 10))
 (segment (start 98.42 82.66) (end 99.255 82.66) (width 0.2) (layer "F.Cu") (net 18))
 (segment (start 89.667 104.7737) (end 87.95 104.7737) (width 0.2) (layer "F.Cu") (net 5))
 (segment (start 90.3937 105.5004) (end 89.667 104.7737) (width 0.2) (layer "F.Cu") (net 5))
 (segment (start 110.5287 106.5237) (end 108.052 104.047) (width 0.2) (layer "F.Cu") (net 5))
 (segment (start 108.052 104.047) (end 95.8631 104.047) (width 0.2) (layer "F.Cu") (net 5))
 (segment (start 94.4097 105.5004) (end 90.3937 105.5004) (width 0.2) (layer "F.Cu") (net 5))
 (segment (start 95.8631 104.047) (end 94.4097 105.5004) (width 0.2) (layer "F.Cu") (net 5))
 (segment (start 128.4483 106.575) (end 127.7216 107.3017) (width 0.2) (layer "F.Cu") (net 3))
 (segment (start 108.1304 105.7817) (end 108.1304 104.7737) (width 0.2) (layer "F.Cu") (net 3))
 (segment (start 107.0287 104.7737) (end 108.1304 104.7737) (width 0.2) (layer "F.Cu") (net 3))
 (segment (start 127.7216 107.3017) (end 109.6504 107.3017) (width 0.2) (layer "F.Cu") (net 3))
 (segment (start 129.55 106.575) (end 128.4483 106.575) (width 0.2) (layer "F.Cu") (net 3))
 (segment (start 109.6504 107.3017) (end 108.1304 105.7817) (width 0.2) (layer "F.Cu") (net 3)))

